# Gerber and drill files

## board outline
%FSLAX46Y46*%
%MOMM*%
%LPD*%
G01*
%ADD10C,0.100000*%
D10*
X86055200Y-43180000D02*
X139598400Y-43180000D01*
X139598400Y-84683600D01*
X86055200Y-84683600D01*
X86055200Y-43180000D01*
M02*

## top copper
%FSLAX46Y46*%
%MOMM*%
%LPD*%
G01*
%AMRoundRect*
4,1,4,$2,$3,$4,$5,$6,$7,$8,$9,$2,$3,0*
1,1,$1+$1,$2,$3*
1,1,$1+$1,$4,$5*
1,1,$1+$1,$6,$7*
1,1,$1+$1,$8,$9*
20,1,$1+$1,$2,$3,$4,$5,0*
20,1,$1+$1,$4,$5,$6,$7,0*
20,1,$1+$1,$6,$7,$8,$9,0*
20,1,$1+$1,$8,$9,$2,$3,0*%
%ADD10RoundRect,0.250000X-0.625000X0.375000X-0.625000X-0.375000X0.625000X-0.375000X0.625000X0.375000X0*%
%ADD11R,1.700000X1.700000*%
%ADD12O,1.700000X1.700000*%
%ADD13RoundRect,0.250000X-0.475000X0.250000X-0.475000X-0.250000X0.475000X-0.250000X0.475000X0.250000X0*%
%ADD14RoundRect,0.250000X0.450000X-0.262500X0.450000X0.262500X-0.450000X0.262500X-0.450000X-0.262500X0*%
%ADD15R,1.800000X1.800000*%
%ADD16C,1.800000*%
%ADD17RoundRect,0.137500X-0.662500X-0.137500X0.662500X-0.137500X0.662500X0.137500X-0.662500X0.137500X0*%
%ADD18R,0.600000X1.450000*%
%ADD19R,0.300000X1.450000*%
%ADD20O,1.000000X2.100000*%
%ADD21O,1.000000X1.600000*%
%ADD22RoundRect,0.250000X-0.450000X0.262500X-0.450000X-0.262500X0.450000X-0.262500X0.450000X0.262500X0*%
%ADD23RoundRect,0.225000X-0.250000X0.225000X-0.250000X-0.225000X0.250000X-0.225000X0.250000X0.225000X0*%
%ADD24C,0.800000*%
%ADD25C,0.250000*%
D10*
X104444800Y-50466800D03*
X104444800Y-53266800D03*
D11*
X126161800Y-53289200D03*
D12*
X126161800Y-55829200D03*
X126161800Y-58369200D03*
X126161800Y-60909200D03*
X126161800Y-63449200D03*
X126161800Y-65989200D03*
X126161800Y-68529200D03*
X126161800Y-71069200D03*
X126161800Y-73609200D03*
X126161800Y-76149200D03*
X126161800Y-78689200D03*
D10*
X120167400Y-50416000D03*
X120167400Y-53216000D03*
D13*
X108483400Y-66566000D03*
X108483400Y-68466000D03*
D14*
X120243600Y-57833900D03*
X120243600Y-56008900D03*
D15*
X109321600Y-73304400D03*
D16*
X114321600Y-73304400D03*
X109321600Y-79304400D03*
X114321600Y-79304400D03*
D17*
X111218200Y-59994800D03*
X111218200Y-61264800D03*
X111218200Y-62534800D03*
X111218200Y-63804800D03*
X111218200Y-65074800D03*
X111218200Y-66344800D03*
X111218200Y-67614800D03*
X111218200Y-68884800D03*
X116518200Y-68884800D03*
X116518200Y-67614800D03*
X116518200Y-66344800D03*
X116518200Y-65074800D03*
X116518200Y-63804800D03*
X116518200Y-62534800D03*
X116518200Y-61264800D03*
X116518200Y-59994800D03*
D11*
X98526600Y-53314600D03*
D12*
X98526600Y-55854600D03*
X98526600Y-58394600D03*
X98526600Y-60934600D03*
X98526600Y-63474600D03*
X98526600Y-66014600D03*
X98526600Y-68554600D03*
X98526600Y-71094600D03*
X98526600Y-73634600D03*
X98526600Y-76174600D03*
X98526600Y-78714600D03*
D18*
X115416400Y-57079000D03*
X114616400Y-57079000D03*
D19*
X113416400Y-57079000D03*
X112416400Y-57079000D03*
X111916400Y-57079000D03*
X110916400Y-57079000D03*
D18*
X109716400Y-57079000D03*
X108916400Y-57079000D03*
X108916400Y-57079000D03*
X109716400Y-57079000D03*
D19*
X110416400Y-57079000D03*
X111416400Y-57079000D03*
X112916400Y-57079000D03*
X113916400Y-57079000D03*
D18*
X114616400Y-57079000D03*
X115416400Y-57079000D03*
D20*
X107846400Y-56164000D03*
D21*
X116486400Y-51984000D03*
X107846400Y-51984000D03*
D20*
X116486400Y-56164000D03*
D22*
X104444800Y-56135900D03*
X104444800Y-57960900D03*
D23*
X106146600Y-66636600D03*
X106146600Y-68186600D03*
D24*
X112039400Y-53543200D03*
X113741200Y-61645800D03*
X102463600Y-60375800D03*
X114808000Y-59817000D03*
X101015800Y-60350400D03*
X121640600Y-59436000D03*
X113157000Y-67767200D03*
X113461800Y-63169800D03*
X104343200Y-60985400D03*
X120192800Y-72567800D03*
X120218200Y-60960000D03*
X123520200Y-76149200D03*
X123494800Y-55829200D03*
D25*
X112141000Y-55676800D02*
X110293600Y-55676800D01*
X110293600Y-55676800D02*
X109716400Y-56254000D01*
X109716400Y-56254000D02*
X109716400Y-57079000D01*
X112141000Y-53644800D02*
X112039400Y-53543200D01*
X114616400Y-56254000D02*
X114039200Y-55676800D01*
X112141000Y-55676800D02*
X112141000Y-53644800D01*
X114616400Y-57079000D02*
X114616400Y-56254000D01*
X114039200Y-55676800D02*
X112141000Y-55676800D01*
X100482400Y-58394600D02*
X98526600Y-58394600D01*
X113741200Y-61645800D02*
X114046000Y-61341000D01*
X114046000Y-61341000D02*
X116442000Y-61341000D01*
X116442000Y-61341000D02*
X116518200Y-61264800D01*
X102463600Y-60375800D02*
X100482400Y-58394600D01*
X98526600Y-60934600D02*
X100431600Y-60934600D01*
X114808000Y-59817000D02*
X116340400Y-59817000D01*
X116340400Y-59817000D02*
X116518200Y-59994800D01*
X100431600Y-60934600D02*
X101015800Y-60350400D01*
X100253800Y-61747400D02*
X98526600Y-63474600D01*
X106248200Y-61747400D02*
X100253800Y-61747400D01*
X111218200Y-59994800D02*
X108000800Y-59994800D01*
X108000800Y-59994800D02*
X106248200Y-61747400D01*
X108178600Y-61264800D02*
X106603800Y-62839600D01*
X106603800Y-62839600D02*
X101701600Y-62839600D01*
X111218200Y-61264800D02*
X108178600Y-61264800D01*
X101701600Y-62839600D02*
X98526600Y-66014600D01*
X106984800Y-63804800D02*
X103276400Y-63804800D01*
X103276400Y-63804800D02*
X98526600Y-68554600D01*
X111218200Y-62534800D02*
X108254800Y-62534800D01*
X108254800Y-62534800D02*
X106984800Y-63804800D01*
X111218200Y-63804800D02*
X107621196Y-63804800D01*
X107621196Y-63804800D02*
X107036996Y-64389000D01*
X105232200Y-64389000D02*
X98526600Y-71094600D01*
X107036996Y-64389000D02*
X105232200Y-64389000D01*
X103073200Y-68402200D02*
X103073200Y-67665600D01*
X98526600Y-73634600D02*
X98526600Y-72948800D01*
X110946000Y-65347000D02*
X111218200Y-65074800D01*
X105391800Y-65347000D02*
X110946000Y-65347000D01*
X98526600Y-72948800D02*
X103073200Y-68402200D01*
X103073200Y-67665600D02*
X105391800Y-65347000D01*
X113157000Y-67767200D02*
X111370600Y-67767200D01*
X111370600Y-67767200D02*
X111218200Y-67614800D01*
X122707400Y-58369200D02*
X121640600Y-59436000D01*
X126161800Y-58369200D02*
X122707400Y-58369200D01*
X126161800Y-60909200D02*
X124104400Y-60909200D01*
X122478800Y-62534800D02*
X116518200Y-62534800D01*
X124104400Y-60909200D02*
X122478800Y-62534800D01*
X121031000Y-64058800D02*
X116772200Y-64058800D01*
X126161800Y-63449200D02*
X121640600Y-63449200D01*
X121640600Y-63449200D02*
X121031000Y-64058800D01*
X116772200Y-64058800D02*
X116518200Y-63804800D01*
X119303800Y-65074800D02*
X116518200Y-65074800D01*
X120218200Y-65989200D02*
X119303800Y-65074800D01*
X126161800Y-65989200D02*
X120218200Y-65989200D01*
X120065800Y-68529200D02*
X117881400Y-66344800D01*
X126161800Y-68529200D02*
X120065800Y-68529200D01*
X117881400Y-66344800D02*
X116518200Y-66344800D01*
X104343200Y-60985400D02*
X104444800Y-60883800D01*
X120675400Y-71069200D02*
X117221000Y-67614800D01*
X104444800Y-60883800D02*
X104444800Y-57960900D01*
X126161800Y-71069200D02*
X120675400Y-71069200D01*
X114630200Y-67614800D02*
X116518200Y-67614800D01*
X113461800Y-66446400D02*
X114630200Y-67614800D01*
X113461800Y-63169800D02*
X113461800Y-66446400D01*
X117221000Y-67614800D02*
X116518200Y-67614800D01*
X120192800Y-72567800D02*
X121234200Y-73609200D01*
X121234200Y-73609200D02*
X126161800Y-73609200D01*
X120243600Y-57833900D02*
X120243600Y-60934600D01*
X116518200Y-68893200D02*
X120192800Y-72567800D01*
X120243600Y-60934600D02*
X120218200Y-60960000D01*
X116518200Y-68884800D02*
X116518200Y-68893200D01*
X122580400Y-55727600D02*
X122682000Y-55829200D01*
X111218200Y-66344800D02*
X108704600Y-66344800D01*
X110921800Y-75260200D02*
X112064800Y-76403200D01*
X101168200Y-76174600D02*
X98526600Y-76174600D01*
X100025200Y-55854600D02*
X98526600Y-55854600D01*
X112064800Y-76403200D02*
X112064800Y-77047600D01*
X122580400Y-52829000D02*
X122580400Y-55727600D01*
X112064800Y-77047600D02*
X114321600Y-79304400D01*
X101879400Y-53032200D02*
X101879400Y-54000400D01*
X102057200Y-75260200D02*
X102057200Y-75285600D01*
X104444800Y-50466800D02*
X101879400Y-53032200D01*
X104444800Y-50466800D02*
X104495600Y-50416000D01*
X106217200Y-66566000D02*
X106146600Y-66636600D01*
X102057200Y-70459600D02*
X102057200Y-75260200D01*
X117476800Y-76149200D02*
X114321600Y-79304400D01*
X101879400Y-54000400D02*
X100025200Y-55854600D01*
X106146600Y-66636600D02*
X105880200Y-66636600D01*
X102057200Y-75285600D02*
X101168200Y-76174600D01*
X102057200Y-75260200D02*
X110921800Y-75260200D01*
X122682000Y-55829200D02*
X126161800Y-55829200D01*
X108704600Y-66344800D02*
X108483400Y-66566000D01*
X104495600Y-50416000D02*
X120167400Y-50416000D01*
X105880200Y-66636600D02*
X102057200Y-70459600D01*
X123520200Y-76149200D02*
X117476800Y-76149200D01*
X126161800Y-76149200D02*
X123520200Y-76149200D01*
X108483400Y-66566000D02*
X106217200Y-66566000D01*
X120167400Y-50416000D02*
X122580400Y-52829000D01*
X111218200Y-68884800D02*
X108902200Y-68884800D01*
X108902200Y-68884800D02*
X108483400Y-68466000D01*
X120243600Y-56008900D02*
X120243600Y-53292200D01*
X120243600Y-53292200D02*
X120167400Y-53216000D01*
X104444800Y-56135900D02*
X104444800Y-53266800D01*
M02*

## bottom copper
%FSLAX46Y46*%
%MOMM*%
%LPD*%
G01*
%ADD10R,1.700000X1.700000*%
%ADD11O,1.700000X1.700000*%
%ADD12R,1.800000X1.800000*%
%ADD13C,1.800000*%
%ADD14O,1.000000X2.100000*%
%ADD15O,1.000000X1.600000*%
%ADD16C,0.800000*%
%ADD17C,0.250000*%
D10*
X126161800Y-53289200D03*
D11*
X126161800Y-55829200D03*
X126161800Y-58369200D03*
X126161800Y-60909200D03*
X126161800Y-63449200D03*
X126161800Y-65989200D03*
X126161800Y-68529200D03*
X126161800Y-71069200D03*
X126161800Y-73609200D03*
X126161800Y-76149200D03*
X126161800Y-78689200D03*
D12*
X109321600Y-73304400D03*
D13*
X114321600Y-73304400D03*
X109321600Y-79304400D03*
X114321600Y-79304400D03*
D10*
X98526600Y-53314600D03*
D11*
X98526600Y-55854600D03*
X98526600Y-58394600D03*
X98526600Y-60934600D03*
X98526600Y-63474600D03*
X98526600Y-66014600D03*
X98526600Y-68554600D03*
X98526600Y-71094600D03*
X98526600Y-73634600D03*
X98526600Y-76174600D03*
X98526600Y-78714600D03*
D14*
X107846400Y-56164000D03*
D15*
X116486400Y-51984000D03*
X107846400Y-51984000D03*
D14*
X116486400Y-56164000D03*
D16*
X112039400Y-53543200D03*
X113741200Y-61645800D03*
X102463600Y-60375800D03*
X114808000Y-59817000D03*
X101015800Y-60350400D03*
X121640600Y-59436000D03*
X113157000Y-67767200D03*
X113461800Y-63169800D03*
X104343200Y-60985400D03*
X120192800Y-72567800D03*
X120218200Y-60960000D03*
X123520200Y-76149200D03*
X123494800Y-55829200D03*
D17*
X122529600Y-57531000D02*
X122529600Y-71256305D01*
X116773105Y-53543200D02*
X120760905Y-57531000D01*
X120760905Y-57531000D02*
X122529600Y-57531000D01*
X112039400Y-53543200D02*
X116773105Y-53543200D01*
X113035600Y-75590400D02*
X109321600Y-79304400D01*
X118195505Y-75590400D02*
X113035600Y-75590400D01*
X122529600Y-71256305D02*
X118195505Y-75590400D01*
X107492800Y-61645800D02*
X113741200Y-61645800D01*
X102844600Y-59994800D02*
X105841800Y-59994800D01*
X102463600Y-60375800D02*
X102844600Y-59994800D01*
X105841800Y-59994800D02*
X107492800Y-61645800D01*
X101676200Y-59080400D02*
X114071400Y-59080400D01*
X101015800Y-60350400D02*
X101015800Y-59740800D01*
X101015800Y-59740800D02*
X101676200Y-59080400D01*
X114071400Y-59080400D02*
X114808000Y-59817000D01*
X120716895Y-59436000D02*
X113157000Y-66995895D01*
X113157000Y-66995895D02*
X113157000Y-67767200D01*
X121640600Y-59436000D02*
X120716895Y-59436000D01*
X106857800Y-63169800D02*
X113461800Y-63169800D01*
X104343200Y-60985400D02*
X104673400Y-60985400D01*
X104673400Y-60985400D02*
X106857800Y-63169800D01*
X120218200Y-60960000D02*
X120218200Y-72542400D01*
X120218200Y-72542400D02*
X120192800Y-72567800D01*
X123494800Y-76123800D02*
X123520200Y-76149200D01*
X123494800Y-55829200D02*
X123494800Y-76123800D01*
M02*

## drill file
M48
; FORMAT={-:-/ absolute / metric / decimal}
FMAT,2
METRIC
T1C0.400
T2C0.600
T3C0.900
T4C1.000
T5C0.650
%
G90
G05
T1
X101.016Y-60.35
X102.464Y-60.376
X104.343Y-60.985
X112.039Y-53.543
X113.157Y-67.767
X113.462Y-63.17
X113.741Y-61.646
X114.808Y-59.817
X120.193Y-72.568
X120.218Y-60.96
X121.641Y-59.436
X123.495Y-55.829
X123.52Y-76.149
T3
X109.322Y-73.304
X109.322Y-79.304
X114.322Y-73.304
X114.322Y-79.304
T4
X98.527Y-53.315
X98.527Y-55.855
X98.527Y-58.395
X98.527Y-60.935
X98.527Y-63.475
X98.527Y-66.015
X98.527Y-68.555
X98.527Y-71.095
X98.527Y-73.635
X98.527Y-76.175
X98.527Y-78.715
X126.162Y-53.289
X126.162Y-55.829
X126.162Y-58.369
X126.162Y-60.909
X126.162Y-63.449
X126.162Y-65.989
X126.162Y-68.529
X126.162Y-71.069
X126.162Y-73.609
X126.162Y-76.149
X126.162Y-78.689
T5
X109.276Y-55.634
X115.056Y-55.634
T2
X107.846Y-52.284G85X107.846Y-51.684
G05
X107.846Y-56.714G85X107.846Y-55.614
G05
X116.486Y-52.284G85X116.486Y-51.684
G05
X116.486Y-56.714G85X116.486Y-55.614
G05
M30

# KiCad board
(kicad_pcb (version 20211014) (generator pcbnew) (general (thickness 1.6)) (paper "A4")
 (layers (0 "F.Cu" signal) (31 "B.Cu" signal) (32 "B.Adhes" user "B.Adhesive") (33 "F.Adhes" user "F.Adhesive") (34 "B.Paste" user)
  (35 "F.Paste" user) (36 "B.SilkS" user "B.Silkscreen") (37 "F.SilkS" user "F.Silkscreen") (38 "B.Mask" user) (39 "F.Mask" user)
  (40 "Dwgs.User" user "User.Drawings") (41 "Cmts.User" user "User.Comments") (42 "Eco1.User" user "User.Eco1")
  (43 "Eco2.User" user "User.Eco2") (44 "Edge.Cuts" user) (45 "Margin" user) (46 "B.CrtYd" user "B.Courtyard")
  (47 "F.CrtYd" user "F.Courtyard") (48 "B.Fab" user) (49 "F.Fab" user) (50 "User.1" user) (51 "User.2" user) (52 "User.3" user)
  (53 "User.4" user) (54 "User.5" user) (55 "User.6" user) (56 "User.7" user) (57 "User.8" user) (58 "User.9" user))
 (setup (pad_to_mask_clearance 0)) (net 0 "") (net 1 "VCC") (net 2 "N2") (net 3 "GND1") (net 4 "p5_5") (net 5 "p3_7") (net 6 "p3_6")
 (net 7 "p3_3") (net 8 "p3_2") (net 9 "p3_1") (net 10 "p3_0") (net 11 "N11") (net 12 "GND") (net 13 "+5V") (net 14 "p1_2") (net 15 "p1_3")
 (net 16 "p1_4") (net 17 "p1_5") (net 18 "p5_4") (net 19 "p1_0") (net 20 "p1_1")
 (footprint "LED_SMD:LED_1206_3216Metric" (layer "F.Cu") (at 104.4448 51.8668 -90)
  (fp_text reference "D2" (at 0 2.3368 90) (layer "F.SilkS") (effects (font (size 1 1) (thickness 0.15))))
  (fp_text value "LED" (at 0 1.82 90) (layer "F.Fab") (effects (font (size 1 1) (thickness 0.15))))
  (pad "1" smd roundrect (at -1.4 0 270) (size 1.25 1.75) (layers "F.Cu" "F.Paste" "F.Mask") (roundrect_rratio 0.2) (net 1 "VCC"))
  (pad "2" smd roundrect (at 1.4 0 270) (size 1.25 1.75) (layers "F.Cu" "F.Paste" "F.Mask") (roundrect_rratio 0.2) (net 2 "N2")))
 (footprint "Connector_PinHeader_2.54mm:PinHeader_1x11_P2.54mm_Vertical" (layer "F.Cu") (at 126.1618 53.2892)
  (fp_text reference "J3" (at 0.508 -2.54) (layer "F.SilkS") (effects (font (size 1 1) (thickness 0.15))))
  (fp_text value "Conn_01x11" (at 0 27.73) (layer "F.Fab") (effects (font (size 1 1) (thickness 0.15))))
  (pad "1" thru_hole rect (at 0 0) (size 1.7 1.7) (drill 1) (layers *.Cu *.Mask) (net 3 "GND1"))
  (pad "2" thru_hole oval (at 0 2.54) (size 1.7 1.7) (drill 1) (layers *.Cu *.Mask) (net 1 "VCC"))
  (pad "3" thru_hole oval (at 0 5.08) (size 1.7 1.7) (drill 1) (layers *.Cu *.Mask) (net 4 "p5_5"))
  (pad "4" thru_hole oval (at 0 7.62) (size 1.7 1.7) (drill 1) (layers *.Cu *.Mask) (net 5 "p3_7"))
  (pad "5" thru_hole oval (at 0 10.16) (size 1.7 1.7) (drill 1) (layers *.Cu *.Mask) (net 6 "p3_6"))
  (pad "6" thru_hole oval (at 0 12.7) (size 1.7 1.7) (drill 1) (layers *.Cu *.Mask) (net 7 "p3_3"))
  (pad "7" thru_hole oval (at 0 15.24) (size 1.7 1.7) (drill 1) (layers *.Cu *.Mask) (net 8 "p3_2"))
  (pad "8" thru_hole oval (at 0 17.78) (size 1.7 1.7) (drill 1) (layers *.Cu *.Mask) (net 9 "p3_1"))
  (pad "9" thru_hole oval (at 0 20.32) (size 1.7 1.7) (drill 1) (layers *.Cu *.Mask) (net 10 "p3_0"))
  (pad "10" thru_hole oval (at 0 22.86) (size 1.7 1.7) (drill 1) (layers *.Cu *.Mask) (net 1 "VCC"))
  (pad "11" thru_hole oval (at 0 25.4) (size 1.7 1.7) (drill 1) (layers *.Cu *.Mask) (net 3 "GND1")))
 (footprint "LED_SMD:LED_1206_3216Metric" (layer "F.Cu") (at 120.1674 51.816 -90)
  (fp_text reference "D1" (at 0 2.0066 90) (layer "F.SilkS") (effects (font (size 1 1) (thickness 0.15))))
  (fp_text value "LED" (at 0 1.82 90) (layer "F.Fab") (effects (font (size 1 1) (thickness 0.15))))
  (pad "1" smd roundrect (at -1.4 0 270) (size 1.25 1.75) (layers "F.Cu" "F.Paste" "F.Mask") (roundrect_rratio 0.2) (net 1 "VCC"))
  (pad "2" smd roundrect (at 1.4 0 270) (size 1.25 1.75) (layers "F.Cu" "F.Paste" "F.Mask") (roundrect_rratio 0.2) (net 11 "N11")))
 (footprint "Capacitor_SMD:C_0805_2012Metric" (layer "F.Cu") (at 108.4834 67.516 -90)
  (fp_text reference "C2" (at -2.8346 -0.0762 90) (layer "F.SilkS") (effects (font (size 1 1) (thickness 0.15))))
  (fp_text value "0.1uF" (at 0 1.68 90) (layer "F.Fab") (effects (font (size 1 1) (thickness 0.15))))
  (pad "1" smd roundrect (at -0.95 0 270) (size 1 1.45) (layers "F.Cu" "F.Paste" "F.Mask") (roundrect_rratio 0.25) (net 1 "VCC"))
  (pad "2" smd roundrect (at 0.95 0 270) (size 1 1.45) (layers "F.Cu" "F.Paste" "F.Mask") (roundrect_rratio 0.25) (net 3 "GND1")))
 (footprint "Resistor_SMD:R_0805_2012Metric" (layer "F.Cu") (at 120.2436 56.9214 90)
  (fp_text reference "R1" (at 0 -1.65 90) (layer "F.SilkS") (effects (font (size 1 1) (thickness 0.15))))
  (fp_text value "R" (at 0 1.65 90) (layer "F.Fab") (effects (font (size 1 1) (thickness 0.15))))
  (pad "1" smd roundrect (at -0.9125 0 90) (size 1.025 1.4) (layers "F.Cu" "F.Paste" "F.Mask") (roundrect_rratio 0.243902) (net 10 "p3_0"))
  (pad "2" smd roundrect (at 0.9125 0 90) (size 1.025 1.4) (layers "F.Cu" "F.Paste" "F.Mask") (roundrect_rratio 0.243902) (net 11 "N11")))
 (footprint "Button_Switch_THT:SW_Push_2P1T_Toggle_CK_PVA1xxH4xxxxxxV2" (layer "F.Cu") (at 109.3216 73.3044)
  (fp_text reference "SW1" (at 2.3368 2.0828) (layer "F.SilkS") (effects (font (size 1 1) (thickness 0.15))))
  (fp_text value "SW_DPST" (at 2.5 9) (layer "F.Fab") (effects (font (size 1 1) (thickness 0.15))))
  (pad "1" thru_hole rect (at 0 0) (size 1.8 1.8) (drill 0.9) (layers *.Cu *.Mask) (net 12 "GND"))
  (pad "2" thru_hole circle (at 5 0) (size 1.8 1.8) (drill 0.9) (layers *.Cu *.Mask) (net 3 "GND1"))
  (pad "3" thru_hole circle (at 0 6) (size 1.8 1.8) (drill 0.9) (layers *.Cu *.Mask) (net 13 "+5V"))
  (pad "4" thru_hole circle (at 5 6) (size 1.8 1.8) (drill 0.9) (layers *.Cu *.Mask) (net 1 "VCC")))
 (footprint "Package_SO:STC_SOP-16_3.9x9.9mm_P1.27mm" (layer "F.Cu") (at 113.8682 64.4398)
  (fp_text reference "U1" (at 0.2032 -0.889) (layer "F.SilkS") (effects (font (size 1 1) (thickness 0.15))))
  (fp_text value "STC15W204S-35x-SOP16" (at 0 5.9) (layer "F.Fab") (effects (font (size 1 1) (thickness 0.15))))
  (pad "1" smd roundrect (at -2.65 -4.445) (size 1.6 0.55) (layers "F.Cu" "F.Paste" "F.Mask") (roundrect_rratio 0.25) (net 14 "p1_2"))
  (pad "2" smd roundrect (at -2.65 -3.175) (size 1.6 0.55) (layers "F.Cu" "F.Paste" "F.Mask") (roundrect_rratio 0.25) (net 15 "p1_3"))
  (pad "3" smd roundrect (at -2.65 -1.905) (size 1.6 0.55) (layers "F.Cu" "F.Paste" "F.Mask") (roundrect_rratio 0.25) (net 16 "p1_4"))
  (pad "4" smd roundrect (at -2.65 -0.635) (size 1.6 0.55) (layers "F.Cu" "F.Paste" "F.Mask") (roundrect_rratio 0.25) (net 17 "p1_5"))
  (pad "5" smd roundrect (at -2.65 0.635) (size 1.6 0.55) (layers "F.Cu" "F.Paste" "F.Mask") (roundrect_rratio 0.25) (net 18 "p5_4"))
  (pad "6" smd roundrect (at -2.65 1.905) (size 1.6 0.55) (layers "F.Cu" "F.Paste" "F.Mask") (roundrect_rratio 0.25) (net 1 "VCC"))
  (pad "7" smd roundrect (at -2.65 3.175) (size 1.6 0.55) (layers "F.Cu" "F.Paste" "F.Mask") (roundrect_rratio 0.25) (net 4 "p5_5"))
  (pad "8" smd roundrect (at -2.65 4.445) (size 1.6 0.55) (layers "F.Cu" "F.Paste" "F.Mask") (roundrect_rratio 0.25) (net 3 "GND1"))
  (pad "9" smd roundrect (at 2.65 4.445) (size 1.6 0.55) (layers "F.Cu" "F.Paste" "F.Mask") (roundrect_rratio 0.25) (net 10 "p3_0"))
  (pad "10" smd roundrect (at 2.65 3.175) (size 1.6 0.55) (layers "F.Cu" "F.Paste" "F.Mask") (roundrect_rratio 0.25) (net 9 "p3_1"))
  (pad "11" smd roundrect (at 2.65 1.905) (size 1.6 0.55) (layers "F.Cu" "F.Paste" "F.Mask") (roundrect_rratio 0.25) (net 8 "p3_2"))
  (pad "12" smd roundrect (at 2.65 0.635) (size 1.6 0.55) (layers "F.Cu" "F.Paste" "F.Mask") (roundrect_rratio 0.25) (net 7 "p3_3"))
  (pad "13" smd roundrect (at 2.65 -0.635) (size 1.6 0.55) (layers "F.Cu" "F.Paste" "F.Mask") (roundrect_rratio 0.25) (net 6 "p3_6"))
  (pad "14" smd roundrect (at 2.65 -1.905) (size 1.6 0.55) (layers "F.Cu" "F.Paste" "F.Mask") (roundrect_rratio 0.25) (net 5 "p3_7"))
  (pad "15" smd roundrect (at 2.65 -3.175) (size 1.6 0.55) (layers "F.Cu" "F.Paste" "F.Mask") (roundrect_rratio 0.25) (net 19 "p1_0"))
  (pad "16" smd roundrect (at 2.65 -4.445) (size 1.6 0.55) (layers "F.Cu" "F.Paste" "F.Mask") (roundrect_rratio 0.25) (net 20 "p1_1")))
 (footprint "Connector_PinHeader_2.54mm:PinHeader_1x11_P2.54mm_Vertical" (layer "F.Cu") (at 98.5266 53.3146)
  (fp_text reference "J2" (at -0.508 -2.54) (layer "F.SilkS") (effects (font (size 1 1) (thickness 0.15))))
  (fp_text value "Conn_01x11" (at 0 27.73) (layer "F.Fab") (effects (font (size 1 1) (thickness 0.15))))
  (pad "1" thru_hole rect (at 0 0) (size 1.7 1.7) (drill 1) (layers *.Cu *.Mask) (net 3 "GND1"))
  (pad "2" thru_hole oval (at 0 2.54) (size 1.7 1.7) (drill 1) (layers *.Cu *.Mask) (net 1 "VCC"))
  (pad "3" thru_hole oval (at 0 5.08) (size 1.7 1.7) (drill 1) (layers *.Cu *.Mask) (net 19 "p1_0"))
  (pad "4" thru_hole oval (at 0 7.62) (size 1.7 1.7) (drill 1) (layers *.Cu *.Mask) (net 20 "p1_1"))
  (pad "5" thru_hole oval (at 0 10.16) (size 1.7 1.7) (drill 1) (layers *.Cu *.Mask) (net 14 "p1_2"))
  (pad "6" thru_hole oval (at 0 12.7) (size 1.7 1.7) (drill 1) (layers *.Cu *.Mask) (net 15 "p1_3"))
  (pad "7" thru_hole oval (at 0 15.24) (size 1.7 1.7) (drill 1) (layers *.Cu *.Mask) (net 16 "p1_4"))
  (pad "8" thru_hole oval (at 0 17.78) (size 1.7 1.7) (drill 1) (layers *.Cu *.Mask) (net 17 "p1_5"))
  (pad "9" thru_hole oval (at 0 20.32) (size 1.7 1.7) (drill 1) (layers *.Cu *.Mask) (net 18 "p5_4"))
  (pad "10" thru_hole oval (at 0 22.86) (size 1.7 1.7) (drill 1) (layers *.Cu *.Mask) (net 1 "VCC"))
  (pad "11" thru_hole oval (at 0 25.4) (size 1.7 1.7) (drill 1) (layers *.Cu *.Mask) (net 3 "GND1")))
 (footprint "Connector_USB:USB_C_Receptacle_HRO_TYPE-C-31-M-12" (layer "F.Cu") (at 112.1664 53.034 180)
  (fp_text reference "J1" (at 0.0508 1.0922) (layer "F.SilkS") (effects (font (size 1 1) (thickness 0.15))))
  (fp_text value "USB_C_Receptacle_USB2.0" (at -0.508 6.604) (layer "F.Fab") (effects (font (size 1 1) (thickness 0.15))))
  (pad "" np_thru_hole circle (at 2.89 -2.6 180) (size 0.65 0.65) (drill 0.65) (layers *.Cu *.Mask))
  (pad "" np_thru_hole circle (at -2.89 -2.6 180) (size 0.65 0.65) (drill 0.65) (layers *.Cu *.Mask))
  (pad "A1" smd rect (at -3.25 -4.045 180) (size 0.6 1.45) (layers "F.Cu" "F.Paste" "F.Mask") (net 12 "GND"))
  (pad "A4" smd rect (at -2.45 -4.045 180) (size 0.6 1.45) (layers "F.Cu" "F.Paste" "F.Mask") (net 13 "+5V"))
  (pad "A5" smd rect (at -1.25 -4.045 180) (size 0.3 1.45) (layers "F.Cu" "F.Paste" "F.Mask") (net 12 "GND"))
  (pad "A6" smd rect (at -0.25 -4.045 180) (size 0.3 1.45) (layers "F.Cu" "F.Paste" "F.Mask") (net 12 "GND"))
  (pad "A7" smd rect (at 0.25 -4.045 180) (size 0.3 1.45) (layers "F.Cu" "F.Paste" "F.Mask") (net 12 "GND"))
  (pad "A8" smd rect (at 1.25 -4.045 180) (size 0.3 1.45) (layers "F.Cu" "F.Paste" "F.Mask") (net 12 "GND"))
  (pad "A9" smd rect (at 2.45 -4.045 180) (size 0.6 1.45) (layers "F.Cu" "F.Paste" "F.Mask") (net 13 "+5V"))
  (pad "A12" smd rect (at 3.25 -4.045 180) (size 0.6 1.45) (layers "F.Cu" "F.Paste" "F.Mask") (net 12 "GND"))
  (pad "B1" smd rect (at 3.25 -4.045 180) (size 0.6 1.45) (layers "F.Cu" "F.Paste" "F.Mask") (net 12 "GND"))
  (pad "B4" smd rect (at 2.45 -4.045 180) (size 0.6 1.45) (layers "F.Cu" "F.Paste" "F.Mask") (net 13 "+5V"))
  (pad "B5" smd rect (at 1.75 -4.045 180) (size 0.3 1.45) (layers "F.Cu" "F.Paste" "F.Mask") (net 12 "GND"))
  (pad "B6" smd rect (at 0.75 -4.045 180) (size 0.3 1.45) (layers "F.Cu" "F.Paste" "F.Mask") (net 12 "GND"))
  (pad "B7" smd rect (at -0.75 -4.045 180) (size 0.3 1.45) (layers "F.Cu" "F.Paste" "F.Mask") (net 12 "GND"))
  (pad "B8" smd rect (at -1.75 -4.045 180) (size 0.3 1.45) (layers "F.Cu" "F.Paste" "F.Mask") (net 12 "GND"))
  (pad "B9" smd rect (at -2.45 -4.045 180) (size 0.6 1.45) (layers "F.Cu" "F.Paste" "F.Mask") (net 13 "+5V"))
  (pad "B12" smd rect (at -3.25 -4.045 180) (size 0.6 1.45) (layers "F.Cu" "F.Paste" "F.Mask") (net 12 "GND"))
  (pad "S1" thru_hole oval (at 4.32 -3.13 180) (size 1 2.1) (drill oval 0.6 1.7) (layers *.Cu *.Mask) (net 12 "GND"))
  (pad "S1" thru_hole oval (at -4.32 1.05 180) (size 1 1.6) (drill oval 0.6 1.2) (layers *.Cu *.Mask) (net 12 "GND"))
  (pad "S1" thru_hole oval (at 4.32 1.05 180) (size 1 1.6) (drill oval 0.6 1.2) (layers *.Cu *.Mask) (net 12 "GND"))
  (pad "S1" thru_hole oval (at -4.32 -3.13 180) (size 1 2.1) (drill oval 0.6 1.7) (layers *.Cu *.Mask) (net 12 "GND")))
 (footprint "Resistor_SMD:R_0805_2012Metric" (layer "F.Cu") (at 104.4448 57.0484 -90)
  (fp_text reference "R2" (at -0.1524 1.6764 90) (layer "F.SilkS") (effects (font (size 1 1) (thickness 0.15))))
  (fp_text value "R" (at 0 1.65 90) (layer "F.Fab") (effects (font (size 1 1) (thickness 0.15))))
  (pad "1" smd roundrect (at -0.9125 0 270) (size 1.025 1.4) (layers "F.Cu" "F.Paste" "F.Mask") (roundrect_rratio 0.243902) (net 2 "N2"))
  (pad "2" smd roundrect (at 0.9125 0 270) (size 1.025 1.4) (layers "F.Cu" "F.Paste" "F.Mask") (roundrect_rratio 0.243902) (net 9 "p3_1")))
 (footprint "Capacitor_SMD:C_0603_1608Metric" (layer "F.Cu") (at 106.1466 67.4116 -90)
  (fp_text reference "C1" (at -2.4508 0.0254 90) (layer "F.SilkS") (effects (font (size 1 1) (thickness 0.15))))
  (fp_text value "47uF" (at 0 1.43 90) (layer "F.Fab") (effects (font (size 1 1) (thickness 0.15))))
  (pad "1" smd roundrect (at -0.775 0 270) (size 0.9 0.95) (layers "F.Cu" "F.Paste" "F.Mask") (roundrect_rratio 0.25) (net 1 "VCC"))
  (pad "2" smd roundrect (at 0.775 0 270) (size 0.9 0.95) (layers "F.Cu" "F.Paste" "F.Mask") (roundrect_rratio 0.25) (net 3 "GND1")))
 (gr_rect (start 86.0552 43.18) (end 139.5984 84.6836) (layer "Edge.Cuts") (width 0.1) (fill none))
 (segment (start 112.141 55.6768) (end 110.2936 55.6768) (width 0.25) (layer "F.Cu") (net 13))
 (segment (start 110.2936 55.6768) (end 109.7164 56.254) (width 0.25) (layer "F.Cu") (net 13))
 (segment (start 109.7164 56.254) (end 109.7164 57.079) (width 0.25) (layer "F.Cu") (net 13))
 (segment (start 112.141 53.6448) (end 112.0394 53.5432) (width 0.25) (layer "F.Cu") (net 13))
 (segment (start 114.6164 56.254) (end 114.0392 55.6768) (width 0.25) (layer "F.Cu") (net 13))
 (segment (start 112.141 55.6768) (end 112.141 53.6448) (width 0.25) (layer "F.Cu") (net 13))
 (segment (start 114.6164 57.079) (end 114.6164 56.254) (width 0.25) (layer "F.Cu") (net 13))
 (segment (start 114.0392 55.6768) (end 112.141 55.6768) (width 0.25) (layer "F.Cu") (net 13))
 (via (at 112.0394 53.5432) (size 0.8) (drill 0.4) (layers "F.Cu" "B.Cu") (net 13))
 (segment (start 122.5296 57.531) (end 122.5296 71.256305) (width 0.25) (layer "B.Cu") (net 13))
 (segment (start 116.773105 53.5432) (end 120.760905 57.531) (width 0.25) (layer "B.Cu") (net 13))
 (segment (start 120.760905 57.531) (end 122.5296 57.531) (width 0.25) (layer "B.Cu") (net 13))
 (segment (start 112.0394 53.5432) (end 116.773105 53.5432) (width 0.25) (layer "B.Cu") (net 13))
 (segment (start 113.0356 75.5904) (end 109.3216 79.3044) (width 0.25) (layer "B.Cu") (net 13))
 (segment (start 118.195505 75.5904) (end 113.0356 75.5904) (width 0.25) (layer "B.Cu") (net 13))
 (segment (start 122.5296 71.256305) (end 118.195505 75.5904) (width 0.25) (layer "B.Cu") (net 13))
 (segment (start 100.4824 58.3946) (end 98.5266 58.3946) (width 0.25) (layer "F.Cu") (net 19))
 (segment (start 113.7412 61.6458) (end 114.046 61.341) (width 0.25) (layer "F.Cu") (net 19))
 (segment (start 114.046 61.341) (end 116.442 61.341) (width 0.25) (layer "F.Cu") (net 19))
 (segment (start 116.442 61.341) (end 116.5182 61.2648) (width 0.25) (layer "F.Cu") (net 19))
 (segment (start 102.4636 60.3758) (end 100.4824 58.3946) (width 0.25) (layer "F.Cu") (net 19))
 (via (at 113.7412 61.6458) (size 0.8) (drill 0.4) (layers "F.Cu" "B.Cu") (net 19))
 (via (at 102.4636 60.3758) (size 0.8) (drill 0.4) (layers "F.Cu" "B.Cu") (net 19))
 (segment (start 107.4928 61.6458) (end 113.7412 61.6458) (width 0.25) (layer "B.Cu") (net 19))
 (segment (start 102.8446 59.9948) (end 105.8418 59.9948) (width 0.25) (layer "B.Cu") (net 19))
 (segment (start 102.4636 60.3758) (end 102.8446 59.9948) (width 0.25) (layer "B.Cu") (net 19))
 (segment (start 105.8418 59.9948) (end 107.4928 61.6458) (width 0.25) (layer "B.Cu") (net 19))
 (segment (start 98.5266 60.9346) (end 100.4316 60.9346) (width 0.25) (layer "F.Cu") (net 20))
 (segment (start 114.808 59.817) (end 116.3404 59.817) (width 0.25) (layer "F.Cu") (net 20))
 (segment (start 116.3404 59.817) (end 116.5182 59.9948) (width 0.25) (layer "F.Cu") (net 20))
 (segment (start 100.4316 60.9346) (end 101.0158 60.3504) (width 0.25) (layer "F.Cu") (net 20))
 (via (at 114.808 59.817) (size 0.8) (drill 0.4) (layers "F.Cu" "B.Cu") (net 20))
 (via (at 101.0158 60.3504) (size 0.8) (drill 0.4) (layers "F.Cu" "B.Cu") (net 20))
 (segment (start 101.6762 59.0804) (end 114.0714 59.0804) (width 0.25) (layer "B.Cu") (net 20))
 (segment (start 101.0158 60.3504) (end 101.0158 59.7408) (width 0.25) (layer "B.Cu") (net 20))
 (segment (start 101.0158 59.7408) (end 101.6762 59.0804) (width 0.25) (layer "B.Cu") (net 20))
 (segment (start 114.0714 59.0804) (end 114.808 59.817) (width 0.25) (layer "B.Cu") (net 20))
 (segment (start 100.2538 61.7474) (end 98.5266 63.4746) (width 0.25) (layer "F.Cu") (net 14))
 (segment (start 106.2482 61.7474) (end 100.2538 61.7474) (width 0.25) (layer "F.Cu") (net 14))
 (segment (start 111.2182 59.9948) (end 108.0008 59.9948) (width 0.25) (layer "F.Cu") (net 14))
 (segment (start 108.0008 59.9948) (end 106.2482 61.7474) (width 0.25) (layer "F.Cu") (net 14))
 (segment (start 108.1786 61.2648) (end 106.6038 62.8396) (width 0.25) (layer "F.Cu") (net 15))
 (segment (start 106.6038 62.8396) (end 101.7016 62.8396) (width 0.25) (layer "F.Cu") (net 15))
 (segment (start 111.2182 61.2648) (end 108.1786 61.2648) (width 0.25) (layer "F.Cu") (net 15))
 (segment (start 101.7016 62.8396) (end 98.5266 66.0146) (width 0.25) (layer "F.Cu") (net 15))
 (segment (start 106.9848 63.8048) (end 103.2764 63.8048) (width 0.25) (layer "F.Cu") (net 16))
 (segment (start 103.2764 63.8048) (end 98.5266 68.5546) (width 0.25) (layer "F.Cu") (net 16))
 (segment (start 111.2182 62.5348) (end 108.2548 62.5348) (width 0.25) (layer "F.Cu") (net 16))
 (segment (start 108.2548 62.5348) (end 106.9848 63.8048) (width 0.25) (layer "F.Cu") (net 16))
 (segment (start 111.2182 63.8048) (end 107.621196 63.8048) (width 0.25) (layer "F.Cu") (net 17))
 (segment (start 107.621196 63.8048) (end 107.036996 64.389) (width 0.25) (layer "F.Cu") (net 17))
 (segment (start 105.2322 64.389) (end 98.5266 71.0946) (width 0.25) (layer "F.Cu") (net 17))
 (segment (start 107.036996 64.389) (end 105.2322 64.389) (width 0.25) (layer "F.Cu") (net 17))
 (segment (start 103.0732 68.4022) (end 103.0732 67.6656) (width 0.25) (layer "F.Cu") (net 18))
 (segment (start 98.5266 73.6346) (end 98.5266 72.9488) (width 0.25) (layer "F.Cu") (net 18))
 (segment (start 110.946 65.347) (end 111.2182 65.0748) (width 0.25) (layer "F.Cu") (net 18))
 (segment (start 105.3918 65.347) (end 110.946 65.347) (width 0.25) (layer "F.Cu") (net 18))
 (segment (start 98.5266 72.9488) (end 103.0732 68.4022) (width 0.25) (layer "F.Cu") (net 18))
 (segment (start 103.0732 67.6656) (end 105.3918 65.347) (width 0.25) (layer "F.Cu") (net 18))
 (segment (start 113.157 67.7672) (end 111.3706 67.7672) (width 0.25) (layer "F.Cu") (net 4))
 (segment (start 111.3706 67.7672) (end 111.2182 67.6148) (width 0.25) (layer "F.Cu") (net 4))
 (segment (start 122.7074 58.3692) (end 121.6406 59.436) (width 0.25) (layer "F.Cu") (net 4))
 (segment (start 126.1618 58.3692) (end 122.7074 58.3692) (width 0.25) (layer "F.Cu") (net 4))
 (via (at 121.6406 59.436) (size 0.8) (drill 0.4) (layers "F.Cu" "B.Cu") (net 4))
 (via (at 113.157 67.7672) (size 0.8) (drill 0.4) (layers "F.Cu" "B.Cu") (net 4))
 (segment (start 120.716895 59.436) (end 113.157 66.995895) (width 0.25) (layer "B.Cu") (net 4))
 (segment (start 113.157 66.995895) (end 113.157 67.7672) (width 0.25) (layer "B.Cu") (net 4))
 (segment (start 121.6406 59.436) (end 120.716895 59.436) (width 0.25) (layer "B.Cu") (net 4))
 (segment (start 126.1618 60.9092) (end 124.1044 60.9092) (width 0.25) (layer "F.Cu") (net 5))
 (segment (start 122.4788 62.5348) (end 116.5182 62.5348) (width 0.25) (layer "F.Cu") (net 5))
 (segment (start 124.1044 60.9092) (end 122.4788 62.5348) (width 0.25) (layer "F.Cu") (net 5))
 (segment (start 121.031 64.0588) (end 116.7722 64.0588) (width 0.25) (layer "F.Cu") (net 6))
 (segment (start 126.1618 63.4492) (end 121.6406 63.4492) (width 0.25) (layer "F.Cu") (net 6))
 (segment (start 121.6406 63.4492) (end 121.031 64.0588) (width 0.25) (layer "F.Cu") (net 6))
 (segment (start 116.7722 64.0588) (end 116.5182 63.8048) (width 0.25) (layer "F.Cu") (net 6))
 (segment (start 119.3038 65.0748) (end 116.5182 65.0748) (width 0.25) (layer "F.Cu") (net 7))
 (segment (start 120.2182 65.9892) (end 119.3038 65.0748) (width 0.25) (layer "F.Cu") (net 7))
 (segment (start 126.1618 65.9892) (end 120.2182 65.9892) (width 0.25) (layer "F.Cu") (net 7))
 (segment (start 120.0658 68.5292) (end 117.8814 66.3448) (width 0.25) (layer "F.Cu") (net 8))
 (segment (start 126.1618 68.5292) (end 120.0658 68.5292) (width 0.25) (layer "F.Cu") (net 8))
 (segment (start 117.8814 66.3448) (end 116.5182 66.3448) (width 0.25) (layer "F.Cu") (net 8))
 (segment (start 104.3432 60.9854) (end 104.4448 60.8838) (width 0.25) (layer "F.Cu") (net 9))
 (segment (start 120.6754 71.0692) (end 117.221 67.6148) (width 0.25) (layer "F.Cu") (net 9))
 (segment (start 104.4448 60.8838) (end 104.4448 57.9609) (width 0.25) (layer "F.Cu") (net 9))
 (segment (start 126.1618 71.0692) (end 120.6754 71.0692) (width 0.25) (layer "F.Cu") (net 9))
 (segment (start 114.6302 67.6148) (end 116.5182 67.6148) (width 0.25) (layer "F.Cu") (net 9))
 (segment (start 113.4618 66.4464) (end 114.6302 67.6148) (width 0.25) (layer "F.Cu") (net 9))
 (segment (start 113.4618 63.1698) (end 113.4618 66.4464) (width 0.25) (layer "F.Cu") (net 9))
 (segment (start 117.221 67.6148) (end 116.5182 67.6148) (width 0.25) (layer "F.Cu") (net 9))
 (via (at 113.4618 63.1698) (size 0.8) (drill 0.4) (layers "F.Cu" "B.Cu") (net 9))
 (via (at 104.3432 60.9854) (size 0.8) (drill 0.4) (layers "F.Cu" "B.Cu") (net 9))
 (segment (start 106.8578 63.1698) (end 113.4618 63.1698) (width 0.25) (layer "B.Cu") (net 9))
 (segment (start 104.3432 60.9854) (end 104.6734 60.9854) (width 0.25) (layer "B.Cu") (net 9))
 (segment (start 104.6734 60.9854) (end 106.8578 63.1698) (width 0.25) (layer "B.Cu") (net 9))
 (segment (start 120.1928 72.5678) (end 121.2342 73.6092) (width 0.25) (layer "F.Cu") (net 10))
 (segment (start 121.2342 73.6092) (end 126.1618 73.6092) (width 0.25) (layer "F.Cu") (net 10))
 (segment (start 120.2436 57.8339) (end 120.2436 60.9346) (width 0.25) (layer "F.Cu") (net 10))
 (segment (start 116.5182 68.8932) (end 120.1928 72.5678) (width 0.25) (layer "F.Cu") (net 10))
 (segment (start 120.2436 60.9346) (end 120.2182 60.96) (width 0.25) (layer "F.Cu") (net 10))
 (segment (start 116.5182 68.8848) (end 116.5182 68.8932) (width 0.25) (layer "F.Cu") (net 10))
 (via (at 120.1928 72.5678) (size 0.8) (drill 0.4) (layers "F.Cu" "B.Cu") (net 10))
 (via (at 120.2182 60.96) (size 0.8) (drill 0.4) (layers "F.Cu" "B.Cu") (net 10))
 (segment (start 120.2182 60.96) (end 120.2182 72.5424) (width 0.25) (layer "B.Cu") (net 10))
 (segment (start 120.2182 72.5424) (end 120.1928 72.5678) (width 0.25) (layer "B.Cu") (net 10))
 (segment (start 122.5804 55.7276) (end 122.682 55.8292) (width 0.25) (layer "F.Cu") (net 1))
 (segment (start 111.2182 66.3448) (end 108.7046 66.3448) (width 0.25) (layer "F.Cu") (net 1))
 (segment (start 110.9218 75.2602) (end 112.0648 76.4032) (width 0.25) (layer "F.Cu") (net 1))
 (segment (start 101.1682 76.1746) (end 98.5266 76.1746) (width 0.25) (layer "F.Cu") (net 1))
 (segment (start 100.0252 55.8546) (end 98.5266 55.8546) (width 0.25) (layer "F.Cu") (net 1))
 (segment (start 112.0648 76.4032) (end 112.0648 77.0476) (width 0.25) (layer "F.Cu") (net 1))
 (segment (start 122.5804 52.829) (end 122.5804 55.7276) (width 0.25) (layer "F.Cu") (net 1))
 (segment (start 112.0648 77.0476) (end 114.3216 79.3044) (width 0.25) (layer "F.Cu") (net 1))
 (segment (start 101.8794 53.0322) (end 101.8794 54.0004) (width 0.25) (layer "F.Cu") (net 1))
 (segment (start 102.0572 75.2602) (end 102.0572 75.2856) (width 0.25) (layer "F.Cu") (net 1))
 (segment (start 104.4448 50.4668) (end 101.8794 53.0322) (width 0.25) (layer "F.Cu") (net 1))
 (segment (start 104.4448 50.4668) (end 104.4956 50.416) (width 0.25) (layer "F.Cu") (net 1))
 (segment (start 106.2172 66.566) (end 106.1466 66.6366) (width 0.25) (layer "F.Cu") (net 1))
 (segment (start 102.0572 70.4596) (end 102.0572 75.2602) (width 0.25) (layer "F.Cu") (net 1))
 (segment (start 117.4768 76.1492) (end 114.3216 79.3044) (width 0.25) (layer "F.Cu") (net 1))
 (segment (start 101.8794 54.0004) (end 100.0252 55.8546) (width 0.25) (layer "F.Cu") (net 1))
 (segment (start 106.1466 66.6366) (end 105.8802 66.6366) (width 0.25) (layer "F.Cu") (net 1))
 (segment (start 102.0572 75.2856) (end 101.1682 76.1746) (width 0.25) (layer "F.Cu") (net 1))
 (segment (start 102.0572 75.2602) (end 110.9218 75.2602) (width 0.25) (layer "F.Cu") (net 1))
 (segment (start 122.682 55.8292) (end 126.1618 55.8292) (width 0.25) (layer "F.Cu") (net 1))
 (segment (start 108.7046 66.3448) (end 108.4834 66.566) (width 0.25) (layer "F.Cu") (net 1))
 (segment (start 104.4956 50.416) (end 120.1674 50.416) (width 0.25) (layer "F.Cu") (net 1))
 (segment (start 105.8802 66.6366) (end 102.0572 70.4596) (width 0.25) (layer "F.Cu") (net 1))
 (segment (start 123.5202 76.1492) (end 117.4768 76.1492) (width 0.25) (layer "F.Cu") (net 1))
 (segment (start 126.1618 76.1492) (end 123.5202 76.1492) (width 0.25) (layer "F.Cu") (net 1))
 (segment (start 108.4834 66.566) (end 106.2172 66.566) (width 0.25) (layer "F.Cu") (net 1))
 (segment (start 120.1674 50.416) (end 122.5804 52.829) (width 0.25) (layer "F.Cu") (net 1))
 (via (at 123.5202 76.1492) (size 0.8) (drill 0.4) (layers "F.Cu" "B.Cu") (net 1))
 (via (at 123.4948 55.8292) (size 0.8) (drill 0.4) (layers "F.Cu" "B.Cu") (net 1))
 (segment (start 123.4948 76.1238) (end 123.5202 76.1492) (width 0.25) (layer "B.Cu") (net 1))
 (segment (start 123.4948 55.8292) (end 123.4948 76.1238) (width 0.25) (layer "B.Cu") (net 1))
 (segment (start 111.2182 68.8848) (end 108.9022 68.8848) (width 0.25) (layer "F.Cu") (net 3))
 (segment (start 108.9022 68.8848) (end 108.4834 68.466) (width 0.25) (layer "F.Cu") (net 3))
 (segment (start 120.2436 56.0089) (end 120.2436 53.2922) (width 0.25) (layer "F.Cu") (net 11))
 (segment (start 120.2436 53.2922) (end 120.1674 53.216) (width 0.25) (layer "F.Cu") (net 11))
 (segment (start 104.4448 56.1359) (end 104.4448 53.2668) (width 0.25) (layer "F.Cu") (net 2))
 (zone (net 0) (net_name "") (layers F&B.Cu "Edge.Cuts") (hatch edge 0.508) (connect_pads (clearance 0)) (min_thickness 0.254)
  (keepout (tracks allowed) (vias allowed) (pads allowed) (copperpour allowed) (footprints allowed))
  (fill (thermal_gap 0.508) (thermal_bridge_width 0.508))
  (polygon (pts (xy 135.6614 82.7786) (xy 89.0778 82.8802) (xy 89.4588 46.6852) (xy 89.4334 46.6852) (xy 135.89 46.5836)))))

